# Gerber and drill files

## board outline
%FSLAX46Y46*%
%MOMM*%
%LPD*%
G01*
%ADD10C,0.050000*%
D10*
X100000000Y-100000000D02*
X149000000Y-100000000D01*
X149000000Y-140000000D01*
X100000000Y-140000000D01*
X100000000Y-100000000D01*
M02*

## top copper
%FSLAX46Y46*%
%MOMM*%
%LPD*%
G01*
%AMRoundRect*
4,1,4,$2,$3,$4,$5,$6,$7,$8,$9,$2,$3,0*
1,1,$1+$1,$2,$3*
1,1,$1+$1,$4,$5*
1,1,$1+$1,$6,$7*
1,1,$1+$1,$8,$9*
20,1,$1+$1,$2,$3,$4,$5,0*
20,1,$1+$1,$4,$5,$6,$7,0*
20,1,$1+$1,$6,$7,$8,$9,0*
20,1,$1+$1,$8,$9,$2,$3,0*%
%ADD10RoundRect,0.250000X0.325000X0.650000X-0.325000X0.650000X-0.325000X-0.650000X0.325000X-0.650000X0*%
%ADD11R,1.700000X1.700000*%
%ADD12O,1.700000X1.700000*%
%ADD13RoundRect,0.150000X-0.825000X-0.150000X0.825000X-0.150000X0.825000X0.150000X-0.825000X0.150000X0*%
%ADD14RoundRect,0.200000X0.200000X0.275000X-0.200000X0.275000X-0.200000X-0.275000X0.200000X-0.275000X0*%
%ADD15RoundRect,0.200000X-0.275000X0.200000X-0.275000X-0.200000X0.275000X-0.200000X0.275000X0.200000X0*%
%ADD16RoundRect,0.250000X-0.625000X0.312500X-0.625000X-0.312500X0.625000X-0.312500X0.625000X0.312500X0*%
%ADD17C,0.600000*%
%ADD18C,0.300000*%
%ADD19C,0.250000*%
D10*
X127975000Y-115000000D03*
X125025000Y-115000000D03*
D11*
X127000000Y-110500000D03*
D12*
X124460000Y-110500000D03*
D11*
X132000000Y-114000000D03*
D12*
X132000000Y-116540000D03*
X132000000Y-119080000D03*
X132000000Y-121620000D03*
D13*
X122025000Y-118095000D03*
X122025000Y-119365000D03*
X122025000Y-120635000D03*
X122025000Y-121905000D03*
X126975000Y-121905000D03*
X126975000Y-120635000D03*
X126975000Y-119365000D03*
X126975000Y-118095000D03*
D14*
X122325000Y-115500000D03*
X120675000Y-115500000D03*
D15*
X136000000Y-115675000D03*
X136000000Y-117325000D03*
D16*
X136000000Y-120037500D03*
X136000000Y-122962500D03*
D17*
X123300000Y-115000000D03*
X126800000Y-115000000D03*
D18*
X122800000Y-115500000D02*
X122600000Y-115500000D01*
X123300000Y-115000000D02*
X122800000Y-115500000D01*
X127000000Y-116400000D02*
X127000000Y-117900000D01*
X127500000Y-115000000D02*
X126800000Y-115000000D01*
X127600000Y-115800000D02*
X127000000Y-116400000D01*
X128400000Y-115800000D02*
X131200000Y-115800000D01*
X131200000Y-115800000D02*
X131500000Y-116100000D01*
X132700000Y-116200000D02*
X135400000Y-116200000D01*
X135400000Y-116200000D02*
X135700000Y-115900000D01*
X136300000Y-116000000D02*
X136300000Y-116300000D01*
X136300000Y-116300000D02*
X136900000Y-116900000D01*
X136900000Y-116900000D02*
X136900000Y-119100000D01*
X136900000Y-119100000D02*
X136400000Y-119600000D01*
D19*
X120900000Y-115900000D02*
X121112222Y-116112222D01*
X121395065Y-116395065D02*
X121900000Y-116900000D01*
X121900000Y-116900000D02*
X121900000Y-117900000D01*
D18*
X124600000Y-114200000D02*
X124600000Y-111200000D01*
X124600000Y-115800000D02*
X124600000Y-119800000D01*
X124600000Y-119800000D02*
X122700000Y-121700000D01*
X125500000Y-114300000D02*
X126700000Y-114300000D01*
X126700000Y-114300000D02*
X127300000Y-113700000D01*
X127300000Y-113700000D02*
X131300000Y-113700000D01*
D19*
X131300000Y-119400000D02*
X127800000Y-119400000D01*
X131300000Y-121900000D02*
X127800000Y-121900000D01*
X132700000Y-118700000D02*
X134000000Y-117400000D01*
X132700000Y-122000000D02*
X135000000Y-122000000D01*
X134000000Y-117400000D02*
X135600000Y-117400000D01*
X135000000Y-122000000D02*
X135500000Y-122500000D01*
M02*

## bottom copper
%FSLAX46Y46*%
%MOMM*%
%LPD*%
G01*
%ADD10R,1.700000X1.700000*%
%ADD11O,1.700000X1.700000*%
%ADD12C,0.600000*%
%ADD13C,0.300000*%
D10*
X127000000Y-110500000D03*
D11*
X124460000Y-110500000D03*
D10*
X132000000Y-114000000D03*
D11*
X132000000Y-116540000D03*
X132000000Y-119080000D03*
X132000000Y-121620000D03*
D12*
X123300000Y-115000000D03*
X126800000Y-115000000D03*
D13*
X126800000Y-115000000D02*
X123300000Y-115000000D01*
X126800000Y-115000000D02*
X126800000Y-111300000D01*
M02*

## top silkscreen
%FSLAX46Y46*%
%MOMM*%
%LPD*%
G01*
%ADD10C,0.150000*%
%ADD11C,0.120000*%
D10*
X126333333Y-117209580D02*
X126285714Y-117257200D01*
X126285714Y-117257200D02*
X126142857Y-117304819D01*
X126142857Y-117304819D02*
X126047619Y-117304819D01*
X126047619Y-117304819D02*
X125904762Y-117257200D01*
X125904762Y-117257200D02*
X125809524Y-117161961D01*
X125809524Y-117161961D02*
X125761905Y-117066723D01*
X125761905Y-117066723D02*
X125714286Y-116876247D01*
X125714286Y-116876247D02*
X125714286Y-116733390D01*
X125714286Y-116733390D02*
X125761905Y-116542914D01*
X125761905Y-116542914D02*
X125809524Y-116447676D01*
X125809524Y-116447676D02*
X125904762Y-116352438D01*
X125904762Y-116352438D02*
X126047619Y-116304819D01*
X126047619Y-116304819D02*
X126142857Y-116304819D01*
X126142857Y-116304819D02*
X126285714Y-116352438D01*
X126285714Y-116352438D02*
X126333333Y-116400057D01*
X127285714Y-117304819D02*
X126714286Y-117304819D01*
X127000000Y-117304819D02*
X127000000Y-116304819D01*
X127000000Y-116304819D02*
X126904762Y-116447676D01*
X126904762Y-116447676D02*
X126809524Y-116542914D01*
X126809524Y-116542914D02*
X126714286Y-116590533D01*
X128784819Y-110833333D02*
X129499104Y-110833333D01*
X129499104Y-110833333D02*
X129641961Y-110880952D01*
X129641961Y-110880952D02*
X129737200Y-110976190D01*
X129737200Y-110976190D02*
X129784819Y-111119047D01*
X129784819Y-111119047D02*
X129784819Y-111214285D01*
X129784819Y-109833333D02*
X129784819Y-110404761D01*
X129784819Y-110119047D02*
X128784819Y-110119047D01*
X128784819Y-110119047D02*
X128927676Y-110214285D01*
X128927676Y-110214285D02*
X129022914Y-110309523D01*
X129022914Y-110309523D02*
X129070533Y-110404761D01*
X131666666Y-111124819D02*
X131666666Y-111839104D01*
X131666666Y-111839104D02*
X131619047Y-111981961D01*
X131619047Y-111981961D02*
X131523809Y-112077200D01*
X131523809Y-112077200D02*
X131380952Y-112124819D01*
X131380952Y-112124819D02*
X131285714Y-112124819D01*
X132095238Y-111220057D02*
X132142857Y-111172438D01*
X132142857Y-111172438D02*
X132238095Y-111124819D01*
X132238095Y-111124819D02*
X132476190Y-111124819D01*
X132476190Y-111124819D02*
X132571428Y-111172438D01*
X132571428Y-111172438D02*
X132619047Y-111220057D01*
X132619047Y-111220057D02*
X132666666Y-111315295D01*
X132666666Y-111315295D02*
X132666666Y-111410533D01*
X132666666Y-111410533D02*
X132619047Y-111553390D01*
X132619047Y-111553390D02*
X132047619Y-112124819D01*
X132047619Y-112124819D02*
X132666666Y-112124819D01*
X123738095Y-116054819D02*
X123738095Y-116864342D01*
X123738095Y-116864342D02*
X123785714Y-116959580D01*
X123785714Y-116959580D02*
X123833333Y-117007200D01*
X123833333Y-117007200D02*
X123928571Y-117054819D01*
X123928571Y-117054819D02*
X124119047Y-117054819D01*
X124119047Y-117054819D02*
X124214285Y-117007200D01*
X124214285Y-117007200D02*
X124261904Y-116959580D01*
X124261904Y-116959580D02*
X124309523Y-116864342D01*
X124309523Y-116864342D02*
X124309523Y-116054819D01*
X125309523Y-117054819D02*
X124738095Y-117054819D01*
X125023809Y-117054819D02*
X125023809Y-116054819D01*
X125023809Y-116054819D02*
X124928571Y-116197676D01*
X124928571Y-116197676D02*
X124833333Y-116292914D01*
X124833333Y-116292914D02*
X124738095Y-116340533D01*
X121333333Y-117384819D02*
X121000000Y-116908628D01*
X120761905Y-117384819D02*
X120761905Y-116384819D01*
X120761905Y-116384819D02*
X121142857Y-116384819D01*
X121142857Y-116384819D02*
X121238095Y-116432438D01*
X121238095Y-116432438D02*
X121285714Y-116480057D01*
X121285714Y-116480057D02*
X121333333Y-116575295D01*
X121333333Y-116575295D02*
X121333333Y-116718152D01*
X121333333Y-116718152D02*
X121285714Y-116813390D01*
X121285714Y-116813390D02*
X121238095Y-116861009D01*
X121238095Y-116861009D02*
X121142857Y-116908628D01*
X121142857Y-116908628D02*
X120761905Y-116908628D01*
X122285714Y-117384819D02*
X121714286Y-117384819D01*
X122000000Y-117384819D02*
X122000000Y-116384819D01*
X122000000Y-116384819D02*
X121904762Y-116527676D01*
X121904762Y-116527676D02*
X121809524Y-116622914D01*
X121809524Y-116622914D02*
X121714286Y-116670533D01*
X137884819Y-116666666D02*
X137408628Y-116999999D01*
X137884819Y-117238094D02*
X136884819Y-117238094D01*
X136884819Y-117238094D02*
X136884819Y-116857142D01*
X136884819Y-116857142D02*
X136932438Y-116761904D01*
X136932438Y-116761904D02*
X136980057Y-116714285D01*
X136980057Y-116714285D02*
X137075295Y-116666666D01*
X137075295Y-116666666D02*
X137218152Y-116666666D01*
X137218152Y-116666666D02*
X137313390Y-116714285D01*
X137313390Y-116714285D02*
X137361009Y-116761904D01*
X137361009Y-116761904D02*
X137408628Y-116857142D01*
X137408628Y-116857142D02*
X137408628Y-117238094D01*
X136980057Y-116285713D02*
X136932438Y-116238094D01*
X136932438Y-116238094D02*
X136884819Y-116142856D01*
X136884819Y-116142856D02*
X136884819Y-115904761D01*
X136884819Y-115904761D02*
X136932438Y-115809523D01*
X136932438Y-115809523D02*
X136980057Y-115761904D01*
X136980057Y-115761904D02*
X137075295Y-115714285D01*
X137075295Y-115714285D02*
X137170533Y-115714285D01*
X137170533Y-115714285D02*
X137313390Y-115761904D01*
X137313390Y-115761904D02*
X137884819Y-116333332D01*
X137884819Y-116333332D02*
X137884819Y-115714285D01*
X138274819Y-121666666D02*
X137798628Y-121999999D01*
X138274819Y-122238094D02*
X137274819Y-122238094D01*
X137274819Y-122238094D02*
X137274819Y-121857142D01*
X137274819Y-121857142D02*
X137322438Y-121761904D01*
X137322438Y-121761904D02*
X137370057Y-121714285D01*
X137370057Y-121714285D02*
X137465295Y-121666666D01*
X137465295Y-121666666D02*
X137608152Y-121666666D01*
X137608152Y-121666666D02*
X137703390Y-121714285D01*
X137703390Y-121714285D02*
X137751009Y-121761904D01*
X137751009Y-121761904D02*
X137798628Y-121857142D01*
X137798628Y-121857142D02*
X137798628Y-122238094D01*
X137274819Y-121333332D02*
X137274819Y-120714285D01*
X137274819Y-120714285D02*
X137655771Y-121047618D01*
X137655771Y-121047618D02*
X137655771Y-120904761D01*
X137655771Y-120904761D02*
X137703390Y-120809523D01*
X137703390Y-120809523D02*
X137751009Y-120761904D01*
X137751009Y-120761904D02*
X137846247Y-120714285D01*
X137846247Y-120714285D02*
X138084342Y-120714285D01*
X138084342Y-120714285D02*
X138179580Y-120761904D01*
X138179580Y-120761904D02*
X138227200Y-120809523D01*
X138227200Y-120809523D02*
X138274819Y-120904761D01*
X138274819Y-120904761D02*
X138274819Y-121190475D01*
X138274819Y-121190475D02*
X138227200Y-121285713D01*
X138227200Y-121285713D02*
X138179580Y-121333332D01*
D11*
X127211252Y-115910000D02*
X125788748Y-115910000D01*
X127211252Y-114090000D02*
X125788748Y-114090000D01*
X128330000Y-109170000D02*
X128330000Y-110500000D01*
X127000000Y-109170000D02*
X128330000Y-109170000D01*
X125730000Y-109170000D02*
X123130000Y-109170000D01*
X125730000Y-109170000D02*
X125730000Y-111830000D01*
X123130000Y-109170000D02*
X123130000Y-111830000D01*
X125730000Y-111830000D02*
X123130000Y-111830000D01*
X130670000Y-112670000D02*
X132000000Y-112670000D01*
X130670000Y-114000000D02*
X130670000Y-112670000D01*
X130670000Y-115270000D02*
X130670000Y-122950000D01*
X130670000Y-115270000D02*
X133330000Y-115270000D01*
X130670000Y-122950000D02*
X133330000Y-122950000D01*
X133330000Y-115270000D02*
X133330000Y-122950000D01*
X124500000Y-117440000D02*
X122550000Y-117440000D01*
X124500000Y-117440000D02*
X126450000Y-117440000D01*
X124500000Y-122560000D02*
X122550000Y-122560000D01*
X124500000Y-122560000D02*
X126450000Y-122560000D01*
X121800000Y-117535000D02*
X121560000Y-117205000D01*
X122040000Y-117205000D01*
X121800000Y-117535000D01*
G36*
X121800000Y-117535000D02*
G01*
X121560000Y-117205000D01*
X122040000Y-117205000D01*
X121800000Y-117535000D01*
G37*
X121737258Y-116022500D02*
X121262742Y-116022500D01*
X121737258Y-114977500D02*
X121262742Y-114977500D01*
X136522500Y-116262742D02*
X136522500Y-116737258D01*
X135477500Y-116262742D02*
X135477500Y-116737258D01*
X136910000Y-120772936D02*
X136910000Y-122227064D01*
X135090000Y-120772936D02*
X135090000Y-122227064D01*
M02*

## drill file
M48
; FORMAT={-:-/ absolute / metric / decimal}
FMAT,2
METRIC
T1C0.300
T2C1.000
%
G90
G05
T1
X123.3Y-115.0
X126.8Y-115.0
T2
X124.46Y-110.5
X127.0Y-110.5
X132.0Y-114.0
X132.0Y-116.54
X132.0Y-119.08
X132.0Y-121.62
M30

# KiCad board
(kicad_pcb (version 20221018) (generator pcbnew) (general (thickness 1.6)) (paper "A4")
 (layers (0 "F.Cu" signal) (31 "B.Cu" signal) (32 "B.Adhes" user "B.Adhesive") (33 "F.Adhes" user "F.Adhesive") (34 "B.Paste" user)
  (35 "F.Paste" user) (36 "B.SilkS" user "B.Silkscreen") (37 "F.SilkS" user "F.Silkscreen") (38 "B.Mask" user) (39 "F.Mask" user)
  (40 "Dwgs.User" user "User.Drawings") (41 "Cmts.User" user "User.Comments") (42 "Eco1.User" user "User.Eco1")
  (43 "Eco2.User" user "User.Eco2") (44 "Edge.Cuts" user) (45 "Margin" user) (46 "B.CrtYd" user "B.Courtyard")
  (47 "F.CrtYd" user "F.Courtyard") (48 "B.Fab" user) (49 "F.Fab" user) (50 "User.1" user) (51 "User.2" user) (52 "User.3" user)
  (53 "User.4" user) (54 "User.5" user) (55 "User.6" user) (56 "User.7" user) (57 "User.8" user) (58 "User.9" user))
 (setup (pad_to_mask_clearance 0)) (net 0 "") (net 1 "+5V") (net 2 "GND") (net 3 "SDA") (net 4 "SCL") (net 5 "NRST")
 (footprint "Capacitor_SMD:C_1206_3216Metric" (layer "F.Cu") (at 126.5 115 180)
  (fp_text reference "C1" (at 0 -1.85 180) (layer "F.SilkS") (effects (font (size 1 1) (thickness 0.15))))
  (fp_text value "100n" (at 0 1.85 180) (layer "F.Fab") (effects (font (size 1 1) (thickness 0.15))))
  (fp_line (start -0.711252 -0.91) (end 0.711252 -0.91) (stroke (width 0.12) (type solid)) (layer "F.SilkS"))
  (fp_line (start -0.711252 0.91) (end 0.711252 0.91) (stroke (width 0.12) (type solid)) (layer "F.SilkS"))
  (pad "1" smd roundrect (at -1.475 0 180) (size 1.15 1.8) (layers "F.Cu" "F.Paste" "F.Mask") (roundrect_rratio 0.217391) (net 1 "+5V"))
  (pad "2" smd roundrect (at 1.475 0 180) (size 1.15 1.8) (layers "F.Cu" "F.Paste" "F.Mask") (roundrect_rratio 0.217391) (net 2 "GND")))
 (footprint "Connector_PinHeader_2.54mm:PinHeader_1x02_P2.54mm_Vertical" (layer "F.Cu") (at 127 110.5 -90)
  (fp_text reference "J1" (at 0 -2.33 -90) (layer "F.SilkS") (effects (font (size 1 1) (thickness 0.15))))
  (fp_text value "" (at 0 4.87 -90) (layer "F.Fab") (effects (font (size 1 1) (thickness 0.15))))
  (fp_line (start -1.33 -1.33) (end 0 -1.33) (stroke (width 0.12) (type solid)) (layer "F.SilkS"))
  (fp_line (start -1.33 0) (end -1.33 -1.33) (stroke (width 0.12) (type solid)) (layer "F.SilkS"))
  (fp_line (start -1.33 1.27) (end -1.33 3.87) (stroke (width 0.12) (type solid)) (layer "F.SilkS"))
  (fp_line (start -1.33 1.27) (end 1.33 1.27) (stroke (width 0.12) (type solid)) (layer "F.SilkS"))
  (fp_line (start -1.33 3.87) (end 1.33 3.87) (stroke (width 0.12) (type solid)) (layer "F.SilkS"))
  (fp_line (start 1.33 1.27) (end 1.33 3.87) (stroke (width 0.12) (type solid)) (layer "F.SilkS"))
  (pad "1" thru_hole rect (at 0 0 270) (size 1.7 1.7) (drill 1) (layers "*.Cu" "*.Mask") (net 1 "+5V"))
  (pad "2" thru_hole oval (at 0 2.54 270) (size 1.7 1.7) (drill 1) (layers "*.Cu" "*.Mask") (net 2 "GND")))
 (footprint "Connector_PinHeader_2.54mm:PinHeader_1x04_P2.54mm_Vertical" (layer "F.Cu") (at 132 114)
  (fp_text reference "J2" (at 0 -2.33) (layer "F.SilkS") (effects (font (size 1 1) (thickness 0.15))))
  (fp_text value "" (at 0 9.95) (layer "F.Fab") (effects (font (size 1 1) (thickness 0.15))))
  (fp_line (start -1.33 -1.33) (end 0 -1.33) (stroke (width 0.12) (type solid)) (layer "F.SilkS"))
  (fp_line (start -1.33 0) (end -1.33 -1.33) (stroke (width 0.12) (type solid)) (layer "F.SilkS"))
  (fp_line (start -1.33 1.27) (end -1.33 8.95) (stroke (width 0.12) (type solid)) (layer "F.SilkS"))
  (fp_line (start -1.33 1.27) (end 1.33 1.27) (stroke (width 0.12) (type solid)) (layer "F.SilkS"))
  (fp_line (start -1.33 8.95) (end 1.33 8.95) (stroke (width 0.12) (type solid)) (layer "F.SilkS"))
  (fp_line (start 1.33 1.27) (end 1.33 8.95) (stroke (width 0.12) (type solid)) (layer "F.SilkS"))
  (pad "1" thru_hole rect (at 0 0) (size 1.7 1.7) (drill 1) (layers "*.Cu" "*.Mask") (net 2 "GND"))
  (pad "2" thru_hole oval (at 0 2.54) (size 1.7 1.7) (drill 1) (layers "*.Cu" "*.Mask") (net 1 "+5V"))
  (pad "3" thru_hole oval (at 0 5.08) (size 1.7 1.7) (drill 1) (layers "*.Cu" "*.Mask") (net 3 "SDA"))
  (pad "4" thru_hole oval (at 0 7.62) (size 1.7 1.7) (drill 1) (layers "*.Cu" "*.Mask") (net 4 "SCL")))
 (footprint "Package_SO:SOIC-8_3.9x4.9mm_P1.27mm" (layer "F.Cu") (at 124.5 120)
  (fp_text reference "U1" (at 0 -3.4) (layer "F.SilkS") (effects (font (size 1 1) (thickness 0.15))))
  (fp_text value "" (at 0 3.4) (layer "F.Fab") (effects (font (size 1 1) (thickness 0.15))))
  (fp_line (start 0 -2.56) (end -1.95 -2.56) (stroke (width 0.12) (type solid)) (layer "F.SilkS"))
  (fp_line (start 0 -2.56) (end 1.95 -2.56) (stroke (width 0.12) (type solid)) (layer "F.SilkS"))
  (fp_line (start 0 2.56) (end -1.95 2.56) (stroke (width 0.12) (type solid)) (layer "F.SilkS"))
  (fp_line (start 0 2.56) (end 1.95 2.56) (stroke (width 0.12) (type solid)) (layer "F.SilkS"))
  (fp_poly
   (pts (xy -2.7 -2.465) (xy -2.94 -2.795) (xy -2.46 -2.795) (xy -2.7 -2.465)) (stroke (width 0.12) (type solid)) (fill solid)
   (layer "F.SilkS"))
  (pad "1" smd roundrect (at -2.475 -1.905) (size 1.95 0.6) (layers "F.Cu" "F.Paste" "F.Mask") (roundrect_rratio 0.25) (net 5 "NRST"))
  (pad "2" smd roundrect (at -2.475 -0.635) (size 1.95 0.6) (layers "F.Cu" "F.Paste" "F.Mask") (roundrect_rratio 0.25))
  (pad "3" smd roundrect (at -2.475 0.635) (size 1.95 0.6) (layers "F.Cu" "F.Paste" "F.Mask") (roundrect_rratio 0.25))
  (pad "4" smd roundrect (at -2.475 1.905) (size 1.95 0.6) (layers "F.Cu" "F.Paste" "F.Mask") (roundrect_rratio 0.25) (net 2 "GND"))
  (pad "5" smd roundrect (at 2.475 1.905) (size 1.95 0.6) (layers "F.Cu" "F.Paste" "F.Mask") (roundrect_rratio 0.25) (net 4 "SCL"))
  (pad "6" smd roundrect (at 2.475 0.635) (size 1.95 0.6) (layers "F.Cu" "F.Paste" "F.Mask") (roundrect_rratio 0.25))
  (pad "7" smd roundrect (at 2.475 -0.635) (size 1.95 0.6) (layers "F.Cu" "F.Paste" "F.Mask") (roundrect_rratio 0.25) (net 3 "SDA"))
  (pad "8" smd roundrect (at 2.475 -1.905) (size 1.95 0.6) (layers "F.Cu" "F.Paste" "F.Mask") (roundrect_rratio 0.25) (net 1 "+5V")))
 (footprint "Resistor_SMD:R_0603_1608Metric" (layer "F.Cu") (at 121.5 115.5 180)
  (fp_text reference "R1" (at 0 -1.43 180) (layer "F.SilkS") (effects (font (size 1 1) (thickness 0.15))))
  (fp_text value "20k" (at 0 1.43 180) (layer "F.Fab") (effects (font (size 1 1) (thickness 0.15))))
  (fp_line (start -0.237258 -0.5225) (end 0.237258 -0.5225) (stroke (width 0.12) (type solid)) (layer "F.SilkS"))
  (fp_line (start -0.237258 0.5225) (end 0.237258 0.5225) (stroke (width 0.12) (type solid)) (layer "F.SilkS"))
  (pad "1" smd roundrect (at -0.825 0 180) (size 0.8 0.95) (layers "F.Cu" "F.Paste" "F.Mask") (roundrect_rratio 0.25) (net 1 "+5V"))
  (pad "2" smd roundrect (at 0.825 0 180) (size 0.8 0.95) (layers "F.Cu" "F.Paste" "F.Mask") (roundrect_rratio 0.25) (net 5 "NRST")))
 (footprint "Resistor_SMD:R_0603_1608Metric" (layer "F.Cu") (at 136 116.5 -90)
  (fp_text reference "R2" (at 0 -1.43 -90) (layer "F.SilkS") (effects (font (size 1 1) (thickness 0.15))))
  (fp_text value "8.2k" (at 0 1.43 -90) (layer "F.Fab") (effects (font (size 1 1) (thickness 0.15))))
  (fp_line (start -0.237258 -0.5225) (end 0.237258 -0.5225) (stroke (width 0.12) (type solid)) (layer "F.SilkS"))
  (fp_line (start -0.237258 0.5225) (end 0.237258 0.5225) (stroke (width 0.12) (type solid)) (layer "F.SilkS"))
  (pad "1" smd roundrect (at -0.825 0 270) (size 0.8 0.95) (layers "F.Cu" "F.Paste" "F.Mask") (roundrect_rratio 0.25) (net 1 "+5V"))
  (pad "2" smd roundrect (at 0.825 0 270) (size 0.8 0.95) (layers "F.Cu" "F.Paste" "F.Mask") (roundrect_rratio 0.25) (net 3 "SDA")))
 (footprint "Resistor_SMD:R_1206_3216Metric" (layer "F.Cu") (at 136 121.5 -90)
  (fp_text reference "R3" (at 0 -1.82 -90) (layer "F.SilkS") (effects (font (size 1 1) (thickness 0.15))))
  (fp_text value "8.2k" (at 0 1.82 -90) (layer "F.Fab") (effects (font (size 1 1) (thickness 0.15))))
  (fp_line (start -0.727064 -0.91) (end 0.727064 -0.91) (stroke (width 0.12) (type solid)) (layer "F.SilkS"))
  (fp_line (start -0.727064 0.91) (end 0.727064 0.91) (stroke (width 0.12) (type solid)) (layer "F.SilkS"))
  (pad "1" smd roundrect (at -1.4625 0 270) (size 1.125 1.75) (layers "F.Cu" "F.Paste" "F.Mask") (roundrect_rratio 0.222222) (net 1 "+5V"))
  (pad "2" smd roundrect (at 1.4625 0 270) (size 1.125 1.75) (layers "F.Cu" "F.Paste" "F.Mask") (roundrect_rratio 0.222222) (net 4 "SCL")))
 (gr_rect (start 100 100) (end 149 140) (stroke (width 0.05) (type default)) (fill none) (layer "Edge.Cuts"))
 (segment (start 122.8 115.5) (end 122.6 115.5) (width 0.3) (layer "F.Cu") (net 1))
 (segment (start 123.3 115) (end 122.8 115.5) (width 0.3) (layer "F.Cu") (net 1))
 (segment (start 127 116.4) (end 127 117.9) (width 0.3) (layer "F.Cu") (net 1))
 (segment (start 127.5 115) (end 126.8 115) (width 0.3) (layer "F.Cu") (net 1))
 (segment (start 127.6 115.8) (end 127 116.4) (width 0.3) (layer "F.Cu") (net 1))
 (segment (start 128.4 115.8) (end 131.2 115.8) (width 0.3) (layer "F.Cu") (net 1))
 (segment (start 131.2 115.8) (end 131.5 116.1) (width 0.3) (layer "F.Cu") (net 1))
 (segment (start 132.7 116.2) (end 135.4 116.2) (width 0.3) (layer "F.Cu") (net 1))
 (segment (start 135.4 116.2) (end 135.7 115.9) (width 0.3) (layer "F.Cu") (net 1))
 (segment (start 136.3 116) (end 136.3 116.3) (width 0.3) (layer "F.Cu") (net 1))
 (segment (start 136.3 116.3) (end 136.9 116.9) (width 0.3) (layer "F.Cu") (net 1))
 (segment (start 136.9 116.9) (end 136.9 119.1) (width 0.3) (layer "F.Cu") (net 1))
 (segment (start 136.9 119.1) (end 136.4 119.6) (width 0.3) (layer "F.Cu") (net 1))
 (via (at 123.3 115) (size 0.6) (drill 0.3) (layers "F.Cu" "B.Cu") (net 1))
 (via (at 126.8 115) (size 0.6) (drill 0.3) (layers "F.Cu" "B.Cu") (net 1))
 (segment (start 120.9 115.9) (end 121.112222 116.112222) (width 0.25) (layer "F.Cu") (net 5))
 (segment (start 121.395065 116.395065) (end 121.9 116.9) (width 0.25) (layer "F.Cu") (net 5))
 (segment (start 121.9 116.9) (end 121.9 117.9) (width 0.25) (layer "F.Cu") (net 5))
 (segment (start 124.6 114.2) (end 124.6 111.2) (width 0.3) (layer "F.Cu") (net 2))
 (segment (start 124.6 115.8) (end 124.6 119.8) (width 0.3) (layer "F.Cu") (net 2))
 (segment (start 124.6 119.8) (end 122.7 121.7) (width 0.3) (layer "F.Cu") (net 2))
 (segment (start 125.5 114.3) (end 126.7 114.3) (width 0.3) (layer "F.Cu") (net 2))
 (segment (start 126.7 114.3) (end 127.3 113.7) (width 0.3) (layer "F.Cu") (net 2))
 (segment (start 126.8 115) (end 123.3 115) (width 0.3) (layer "B.Cu") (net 1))
 (segment (start 126.8 115) (end 126.8 111.3) (width 0.3) (layer "B.Cu") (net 1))
 (segment (start 127.3 113.7) (end 131.3 113.7) (width 0.3) (layer "F.Cu") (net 2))
 (segment (start 131.3 119.4) (end 127.8 119.4) (width 0.25) (layer "F.Cu") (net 3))
 (segment (start 131.3 121.9) (end 127.8 121.9) (width 0.25) (layer "F.Cu") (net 4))
 (segment (start 132.7 118.7) (end 134 117.4) (width 0.25) (layer "F.Cu") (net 3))
 (segment (start 132.7 122) (end 135 122) (width 0.25) (layer "F.Cu") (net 4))
 (segment (start 134 117.4) (end 135.6 117.4) (width 0.25) (layer "F.Cu") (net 3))
 (segment (start 135 122) (end 135.5 122.5) (width 0.25) (layer "F.Cu") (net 4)))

